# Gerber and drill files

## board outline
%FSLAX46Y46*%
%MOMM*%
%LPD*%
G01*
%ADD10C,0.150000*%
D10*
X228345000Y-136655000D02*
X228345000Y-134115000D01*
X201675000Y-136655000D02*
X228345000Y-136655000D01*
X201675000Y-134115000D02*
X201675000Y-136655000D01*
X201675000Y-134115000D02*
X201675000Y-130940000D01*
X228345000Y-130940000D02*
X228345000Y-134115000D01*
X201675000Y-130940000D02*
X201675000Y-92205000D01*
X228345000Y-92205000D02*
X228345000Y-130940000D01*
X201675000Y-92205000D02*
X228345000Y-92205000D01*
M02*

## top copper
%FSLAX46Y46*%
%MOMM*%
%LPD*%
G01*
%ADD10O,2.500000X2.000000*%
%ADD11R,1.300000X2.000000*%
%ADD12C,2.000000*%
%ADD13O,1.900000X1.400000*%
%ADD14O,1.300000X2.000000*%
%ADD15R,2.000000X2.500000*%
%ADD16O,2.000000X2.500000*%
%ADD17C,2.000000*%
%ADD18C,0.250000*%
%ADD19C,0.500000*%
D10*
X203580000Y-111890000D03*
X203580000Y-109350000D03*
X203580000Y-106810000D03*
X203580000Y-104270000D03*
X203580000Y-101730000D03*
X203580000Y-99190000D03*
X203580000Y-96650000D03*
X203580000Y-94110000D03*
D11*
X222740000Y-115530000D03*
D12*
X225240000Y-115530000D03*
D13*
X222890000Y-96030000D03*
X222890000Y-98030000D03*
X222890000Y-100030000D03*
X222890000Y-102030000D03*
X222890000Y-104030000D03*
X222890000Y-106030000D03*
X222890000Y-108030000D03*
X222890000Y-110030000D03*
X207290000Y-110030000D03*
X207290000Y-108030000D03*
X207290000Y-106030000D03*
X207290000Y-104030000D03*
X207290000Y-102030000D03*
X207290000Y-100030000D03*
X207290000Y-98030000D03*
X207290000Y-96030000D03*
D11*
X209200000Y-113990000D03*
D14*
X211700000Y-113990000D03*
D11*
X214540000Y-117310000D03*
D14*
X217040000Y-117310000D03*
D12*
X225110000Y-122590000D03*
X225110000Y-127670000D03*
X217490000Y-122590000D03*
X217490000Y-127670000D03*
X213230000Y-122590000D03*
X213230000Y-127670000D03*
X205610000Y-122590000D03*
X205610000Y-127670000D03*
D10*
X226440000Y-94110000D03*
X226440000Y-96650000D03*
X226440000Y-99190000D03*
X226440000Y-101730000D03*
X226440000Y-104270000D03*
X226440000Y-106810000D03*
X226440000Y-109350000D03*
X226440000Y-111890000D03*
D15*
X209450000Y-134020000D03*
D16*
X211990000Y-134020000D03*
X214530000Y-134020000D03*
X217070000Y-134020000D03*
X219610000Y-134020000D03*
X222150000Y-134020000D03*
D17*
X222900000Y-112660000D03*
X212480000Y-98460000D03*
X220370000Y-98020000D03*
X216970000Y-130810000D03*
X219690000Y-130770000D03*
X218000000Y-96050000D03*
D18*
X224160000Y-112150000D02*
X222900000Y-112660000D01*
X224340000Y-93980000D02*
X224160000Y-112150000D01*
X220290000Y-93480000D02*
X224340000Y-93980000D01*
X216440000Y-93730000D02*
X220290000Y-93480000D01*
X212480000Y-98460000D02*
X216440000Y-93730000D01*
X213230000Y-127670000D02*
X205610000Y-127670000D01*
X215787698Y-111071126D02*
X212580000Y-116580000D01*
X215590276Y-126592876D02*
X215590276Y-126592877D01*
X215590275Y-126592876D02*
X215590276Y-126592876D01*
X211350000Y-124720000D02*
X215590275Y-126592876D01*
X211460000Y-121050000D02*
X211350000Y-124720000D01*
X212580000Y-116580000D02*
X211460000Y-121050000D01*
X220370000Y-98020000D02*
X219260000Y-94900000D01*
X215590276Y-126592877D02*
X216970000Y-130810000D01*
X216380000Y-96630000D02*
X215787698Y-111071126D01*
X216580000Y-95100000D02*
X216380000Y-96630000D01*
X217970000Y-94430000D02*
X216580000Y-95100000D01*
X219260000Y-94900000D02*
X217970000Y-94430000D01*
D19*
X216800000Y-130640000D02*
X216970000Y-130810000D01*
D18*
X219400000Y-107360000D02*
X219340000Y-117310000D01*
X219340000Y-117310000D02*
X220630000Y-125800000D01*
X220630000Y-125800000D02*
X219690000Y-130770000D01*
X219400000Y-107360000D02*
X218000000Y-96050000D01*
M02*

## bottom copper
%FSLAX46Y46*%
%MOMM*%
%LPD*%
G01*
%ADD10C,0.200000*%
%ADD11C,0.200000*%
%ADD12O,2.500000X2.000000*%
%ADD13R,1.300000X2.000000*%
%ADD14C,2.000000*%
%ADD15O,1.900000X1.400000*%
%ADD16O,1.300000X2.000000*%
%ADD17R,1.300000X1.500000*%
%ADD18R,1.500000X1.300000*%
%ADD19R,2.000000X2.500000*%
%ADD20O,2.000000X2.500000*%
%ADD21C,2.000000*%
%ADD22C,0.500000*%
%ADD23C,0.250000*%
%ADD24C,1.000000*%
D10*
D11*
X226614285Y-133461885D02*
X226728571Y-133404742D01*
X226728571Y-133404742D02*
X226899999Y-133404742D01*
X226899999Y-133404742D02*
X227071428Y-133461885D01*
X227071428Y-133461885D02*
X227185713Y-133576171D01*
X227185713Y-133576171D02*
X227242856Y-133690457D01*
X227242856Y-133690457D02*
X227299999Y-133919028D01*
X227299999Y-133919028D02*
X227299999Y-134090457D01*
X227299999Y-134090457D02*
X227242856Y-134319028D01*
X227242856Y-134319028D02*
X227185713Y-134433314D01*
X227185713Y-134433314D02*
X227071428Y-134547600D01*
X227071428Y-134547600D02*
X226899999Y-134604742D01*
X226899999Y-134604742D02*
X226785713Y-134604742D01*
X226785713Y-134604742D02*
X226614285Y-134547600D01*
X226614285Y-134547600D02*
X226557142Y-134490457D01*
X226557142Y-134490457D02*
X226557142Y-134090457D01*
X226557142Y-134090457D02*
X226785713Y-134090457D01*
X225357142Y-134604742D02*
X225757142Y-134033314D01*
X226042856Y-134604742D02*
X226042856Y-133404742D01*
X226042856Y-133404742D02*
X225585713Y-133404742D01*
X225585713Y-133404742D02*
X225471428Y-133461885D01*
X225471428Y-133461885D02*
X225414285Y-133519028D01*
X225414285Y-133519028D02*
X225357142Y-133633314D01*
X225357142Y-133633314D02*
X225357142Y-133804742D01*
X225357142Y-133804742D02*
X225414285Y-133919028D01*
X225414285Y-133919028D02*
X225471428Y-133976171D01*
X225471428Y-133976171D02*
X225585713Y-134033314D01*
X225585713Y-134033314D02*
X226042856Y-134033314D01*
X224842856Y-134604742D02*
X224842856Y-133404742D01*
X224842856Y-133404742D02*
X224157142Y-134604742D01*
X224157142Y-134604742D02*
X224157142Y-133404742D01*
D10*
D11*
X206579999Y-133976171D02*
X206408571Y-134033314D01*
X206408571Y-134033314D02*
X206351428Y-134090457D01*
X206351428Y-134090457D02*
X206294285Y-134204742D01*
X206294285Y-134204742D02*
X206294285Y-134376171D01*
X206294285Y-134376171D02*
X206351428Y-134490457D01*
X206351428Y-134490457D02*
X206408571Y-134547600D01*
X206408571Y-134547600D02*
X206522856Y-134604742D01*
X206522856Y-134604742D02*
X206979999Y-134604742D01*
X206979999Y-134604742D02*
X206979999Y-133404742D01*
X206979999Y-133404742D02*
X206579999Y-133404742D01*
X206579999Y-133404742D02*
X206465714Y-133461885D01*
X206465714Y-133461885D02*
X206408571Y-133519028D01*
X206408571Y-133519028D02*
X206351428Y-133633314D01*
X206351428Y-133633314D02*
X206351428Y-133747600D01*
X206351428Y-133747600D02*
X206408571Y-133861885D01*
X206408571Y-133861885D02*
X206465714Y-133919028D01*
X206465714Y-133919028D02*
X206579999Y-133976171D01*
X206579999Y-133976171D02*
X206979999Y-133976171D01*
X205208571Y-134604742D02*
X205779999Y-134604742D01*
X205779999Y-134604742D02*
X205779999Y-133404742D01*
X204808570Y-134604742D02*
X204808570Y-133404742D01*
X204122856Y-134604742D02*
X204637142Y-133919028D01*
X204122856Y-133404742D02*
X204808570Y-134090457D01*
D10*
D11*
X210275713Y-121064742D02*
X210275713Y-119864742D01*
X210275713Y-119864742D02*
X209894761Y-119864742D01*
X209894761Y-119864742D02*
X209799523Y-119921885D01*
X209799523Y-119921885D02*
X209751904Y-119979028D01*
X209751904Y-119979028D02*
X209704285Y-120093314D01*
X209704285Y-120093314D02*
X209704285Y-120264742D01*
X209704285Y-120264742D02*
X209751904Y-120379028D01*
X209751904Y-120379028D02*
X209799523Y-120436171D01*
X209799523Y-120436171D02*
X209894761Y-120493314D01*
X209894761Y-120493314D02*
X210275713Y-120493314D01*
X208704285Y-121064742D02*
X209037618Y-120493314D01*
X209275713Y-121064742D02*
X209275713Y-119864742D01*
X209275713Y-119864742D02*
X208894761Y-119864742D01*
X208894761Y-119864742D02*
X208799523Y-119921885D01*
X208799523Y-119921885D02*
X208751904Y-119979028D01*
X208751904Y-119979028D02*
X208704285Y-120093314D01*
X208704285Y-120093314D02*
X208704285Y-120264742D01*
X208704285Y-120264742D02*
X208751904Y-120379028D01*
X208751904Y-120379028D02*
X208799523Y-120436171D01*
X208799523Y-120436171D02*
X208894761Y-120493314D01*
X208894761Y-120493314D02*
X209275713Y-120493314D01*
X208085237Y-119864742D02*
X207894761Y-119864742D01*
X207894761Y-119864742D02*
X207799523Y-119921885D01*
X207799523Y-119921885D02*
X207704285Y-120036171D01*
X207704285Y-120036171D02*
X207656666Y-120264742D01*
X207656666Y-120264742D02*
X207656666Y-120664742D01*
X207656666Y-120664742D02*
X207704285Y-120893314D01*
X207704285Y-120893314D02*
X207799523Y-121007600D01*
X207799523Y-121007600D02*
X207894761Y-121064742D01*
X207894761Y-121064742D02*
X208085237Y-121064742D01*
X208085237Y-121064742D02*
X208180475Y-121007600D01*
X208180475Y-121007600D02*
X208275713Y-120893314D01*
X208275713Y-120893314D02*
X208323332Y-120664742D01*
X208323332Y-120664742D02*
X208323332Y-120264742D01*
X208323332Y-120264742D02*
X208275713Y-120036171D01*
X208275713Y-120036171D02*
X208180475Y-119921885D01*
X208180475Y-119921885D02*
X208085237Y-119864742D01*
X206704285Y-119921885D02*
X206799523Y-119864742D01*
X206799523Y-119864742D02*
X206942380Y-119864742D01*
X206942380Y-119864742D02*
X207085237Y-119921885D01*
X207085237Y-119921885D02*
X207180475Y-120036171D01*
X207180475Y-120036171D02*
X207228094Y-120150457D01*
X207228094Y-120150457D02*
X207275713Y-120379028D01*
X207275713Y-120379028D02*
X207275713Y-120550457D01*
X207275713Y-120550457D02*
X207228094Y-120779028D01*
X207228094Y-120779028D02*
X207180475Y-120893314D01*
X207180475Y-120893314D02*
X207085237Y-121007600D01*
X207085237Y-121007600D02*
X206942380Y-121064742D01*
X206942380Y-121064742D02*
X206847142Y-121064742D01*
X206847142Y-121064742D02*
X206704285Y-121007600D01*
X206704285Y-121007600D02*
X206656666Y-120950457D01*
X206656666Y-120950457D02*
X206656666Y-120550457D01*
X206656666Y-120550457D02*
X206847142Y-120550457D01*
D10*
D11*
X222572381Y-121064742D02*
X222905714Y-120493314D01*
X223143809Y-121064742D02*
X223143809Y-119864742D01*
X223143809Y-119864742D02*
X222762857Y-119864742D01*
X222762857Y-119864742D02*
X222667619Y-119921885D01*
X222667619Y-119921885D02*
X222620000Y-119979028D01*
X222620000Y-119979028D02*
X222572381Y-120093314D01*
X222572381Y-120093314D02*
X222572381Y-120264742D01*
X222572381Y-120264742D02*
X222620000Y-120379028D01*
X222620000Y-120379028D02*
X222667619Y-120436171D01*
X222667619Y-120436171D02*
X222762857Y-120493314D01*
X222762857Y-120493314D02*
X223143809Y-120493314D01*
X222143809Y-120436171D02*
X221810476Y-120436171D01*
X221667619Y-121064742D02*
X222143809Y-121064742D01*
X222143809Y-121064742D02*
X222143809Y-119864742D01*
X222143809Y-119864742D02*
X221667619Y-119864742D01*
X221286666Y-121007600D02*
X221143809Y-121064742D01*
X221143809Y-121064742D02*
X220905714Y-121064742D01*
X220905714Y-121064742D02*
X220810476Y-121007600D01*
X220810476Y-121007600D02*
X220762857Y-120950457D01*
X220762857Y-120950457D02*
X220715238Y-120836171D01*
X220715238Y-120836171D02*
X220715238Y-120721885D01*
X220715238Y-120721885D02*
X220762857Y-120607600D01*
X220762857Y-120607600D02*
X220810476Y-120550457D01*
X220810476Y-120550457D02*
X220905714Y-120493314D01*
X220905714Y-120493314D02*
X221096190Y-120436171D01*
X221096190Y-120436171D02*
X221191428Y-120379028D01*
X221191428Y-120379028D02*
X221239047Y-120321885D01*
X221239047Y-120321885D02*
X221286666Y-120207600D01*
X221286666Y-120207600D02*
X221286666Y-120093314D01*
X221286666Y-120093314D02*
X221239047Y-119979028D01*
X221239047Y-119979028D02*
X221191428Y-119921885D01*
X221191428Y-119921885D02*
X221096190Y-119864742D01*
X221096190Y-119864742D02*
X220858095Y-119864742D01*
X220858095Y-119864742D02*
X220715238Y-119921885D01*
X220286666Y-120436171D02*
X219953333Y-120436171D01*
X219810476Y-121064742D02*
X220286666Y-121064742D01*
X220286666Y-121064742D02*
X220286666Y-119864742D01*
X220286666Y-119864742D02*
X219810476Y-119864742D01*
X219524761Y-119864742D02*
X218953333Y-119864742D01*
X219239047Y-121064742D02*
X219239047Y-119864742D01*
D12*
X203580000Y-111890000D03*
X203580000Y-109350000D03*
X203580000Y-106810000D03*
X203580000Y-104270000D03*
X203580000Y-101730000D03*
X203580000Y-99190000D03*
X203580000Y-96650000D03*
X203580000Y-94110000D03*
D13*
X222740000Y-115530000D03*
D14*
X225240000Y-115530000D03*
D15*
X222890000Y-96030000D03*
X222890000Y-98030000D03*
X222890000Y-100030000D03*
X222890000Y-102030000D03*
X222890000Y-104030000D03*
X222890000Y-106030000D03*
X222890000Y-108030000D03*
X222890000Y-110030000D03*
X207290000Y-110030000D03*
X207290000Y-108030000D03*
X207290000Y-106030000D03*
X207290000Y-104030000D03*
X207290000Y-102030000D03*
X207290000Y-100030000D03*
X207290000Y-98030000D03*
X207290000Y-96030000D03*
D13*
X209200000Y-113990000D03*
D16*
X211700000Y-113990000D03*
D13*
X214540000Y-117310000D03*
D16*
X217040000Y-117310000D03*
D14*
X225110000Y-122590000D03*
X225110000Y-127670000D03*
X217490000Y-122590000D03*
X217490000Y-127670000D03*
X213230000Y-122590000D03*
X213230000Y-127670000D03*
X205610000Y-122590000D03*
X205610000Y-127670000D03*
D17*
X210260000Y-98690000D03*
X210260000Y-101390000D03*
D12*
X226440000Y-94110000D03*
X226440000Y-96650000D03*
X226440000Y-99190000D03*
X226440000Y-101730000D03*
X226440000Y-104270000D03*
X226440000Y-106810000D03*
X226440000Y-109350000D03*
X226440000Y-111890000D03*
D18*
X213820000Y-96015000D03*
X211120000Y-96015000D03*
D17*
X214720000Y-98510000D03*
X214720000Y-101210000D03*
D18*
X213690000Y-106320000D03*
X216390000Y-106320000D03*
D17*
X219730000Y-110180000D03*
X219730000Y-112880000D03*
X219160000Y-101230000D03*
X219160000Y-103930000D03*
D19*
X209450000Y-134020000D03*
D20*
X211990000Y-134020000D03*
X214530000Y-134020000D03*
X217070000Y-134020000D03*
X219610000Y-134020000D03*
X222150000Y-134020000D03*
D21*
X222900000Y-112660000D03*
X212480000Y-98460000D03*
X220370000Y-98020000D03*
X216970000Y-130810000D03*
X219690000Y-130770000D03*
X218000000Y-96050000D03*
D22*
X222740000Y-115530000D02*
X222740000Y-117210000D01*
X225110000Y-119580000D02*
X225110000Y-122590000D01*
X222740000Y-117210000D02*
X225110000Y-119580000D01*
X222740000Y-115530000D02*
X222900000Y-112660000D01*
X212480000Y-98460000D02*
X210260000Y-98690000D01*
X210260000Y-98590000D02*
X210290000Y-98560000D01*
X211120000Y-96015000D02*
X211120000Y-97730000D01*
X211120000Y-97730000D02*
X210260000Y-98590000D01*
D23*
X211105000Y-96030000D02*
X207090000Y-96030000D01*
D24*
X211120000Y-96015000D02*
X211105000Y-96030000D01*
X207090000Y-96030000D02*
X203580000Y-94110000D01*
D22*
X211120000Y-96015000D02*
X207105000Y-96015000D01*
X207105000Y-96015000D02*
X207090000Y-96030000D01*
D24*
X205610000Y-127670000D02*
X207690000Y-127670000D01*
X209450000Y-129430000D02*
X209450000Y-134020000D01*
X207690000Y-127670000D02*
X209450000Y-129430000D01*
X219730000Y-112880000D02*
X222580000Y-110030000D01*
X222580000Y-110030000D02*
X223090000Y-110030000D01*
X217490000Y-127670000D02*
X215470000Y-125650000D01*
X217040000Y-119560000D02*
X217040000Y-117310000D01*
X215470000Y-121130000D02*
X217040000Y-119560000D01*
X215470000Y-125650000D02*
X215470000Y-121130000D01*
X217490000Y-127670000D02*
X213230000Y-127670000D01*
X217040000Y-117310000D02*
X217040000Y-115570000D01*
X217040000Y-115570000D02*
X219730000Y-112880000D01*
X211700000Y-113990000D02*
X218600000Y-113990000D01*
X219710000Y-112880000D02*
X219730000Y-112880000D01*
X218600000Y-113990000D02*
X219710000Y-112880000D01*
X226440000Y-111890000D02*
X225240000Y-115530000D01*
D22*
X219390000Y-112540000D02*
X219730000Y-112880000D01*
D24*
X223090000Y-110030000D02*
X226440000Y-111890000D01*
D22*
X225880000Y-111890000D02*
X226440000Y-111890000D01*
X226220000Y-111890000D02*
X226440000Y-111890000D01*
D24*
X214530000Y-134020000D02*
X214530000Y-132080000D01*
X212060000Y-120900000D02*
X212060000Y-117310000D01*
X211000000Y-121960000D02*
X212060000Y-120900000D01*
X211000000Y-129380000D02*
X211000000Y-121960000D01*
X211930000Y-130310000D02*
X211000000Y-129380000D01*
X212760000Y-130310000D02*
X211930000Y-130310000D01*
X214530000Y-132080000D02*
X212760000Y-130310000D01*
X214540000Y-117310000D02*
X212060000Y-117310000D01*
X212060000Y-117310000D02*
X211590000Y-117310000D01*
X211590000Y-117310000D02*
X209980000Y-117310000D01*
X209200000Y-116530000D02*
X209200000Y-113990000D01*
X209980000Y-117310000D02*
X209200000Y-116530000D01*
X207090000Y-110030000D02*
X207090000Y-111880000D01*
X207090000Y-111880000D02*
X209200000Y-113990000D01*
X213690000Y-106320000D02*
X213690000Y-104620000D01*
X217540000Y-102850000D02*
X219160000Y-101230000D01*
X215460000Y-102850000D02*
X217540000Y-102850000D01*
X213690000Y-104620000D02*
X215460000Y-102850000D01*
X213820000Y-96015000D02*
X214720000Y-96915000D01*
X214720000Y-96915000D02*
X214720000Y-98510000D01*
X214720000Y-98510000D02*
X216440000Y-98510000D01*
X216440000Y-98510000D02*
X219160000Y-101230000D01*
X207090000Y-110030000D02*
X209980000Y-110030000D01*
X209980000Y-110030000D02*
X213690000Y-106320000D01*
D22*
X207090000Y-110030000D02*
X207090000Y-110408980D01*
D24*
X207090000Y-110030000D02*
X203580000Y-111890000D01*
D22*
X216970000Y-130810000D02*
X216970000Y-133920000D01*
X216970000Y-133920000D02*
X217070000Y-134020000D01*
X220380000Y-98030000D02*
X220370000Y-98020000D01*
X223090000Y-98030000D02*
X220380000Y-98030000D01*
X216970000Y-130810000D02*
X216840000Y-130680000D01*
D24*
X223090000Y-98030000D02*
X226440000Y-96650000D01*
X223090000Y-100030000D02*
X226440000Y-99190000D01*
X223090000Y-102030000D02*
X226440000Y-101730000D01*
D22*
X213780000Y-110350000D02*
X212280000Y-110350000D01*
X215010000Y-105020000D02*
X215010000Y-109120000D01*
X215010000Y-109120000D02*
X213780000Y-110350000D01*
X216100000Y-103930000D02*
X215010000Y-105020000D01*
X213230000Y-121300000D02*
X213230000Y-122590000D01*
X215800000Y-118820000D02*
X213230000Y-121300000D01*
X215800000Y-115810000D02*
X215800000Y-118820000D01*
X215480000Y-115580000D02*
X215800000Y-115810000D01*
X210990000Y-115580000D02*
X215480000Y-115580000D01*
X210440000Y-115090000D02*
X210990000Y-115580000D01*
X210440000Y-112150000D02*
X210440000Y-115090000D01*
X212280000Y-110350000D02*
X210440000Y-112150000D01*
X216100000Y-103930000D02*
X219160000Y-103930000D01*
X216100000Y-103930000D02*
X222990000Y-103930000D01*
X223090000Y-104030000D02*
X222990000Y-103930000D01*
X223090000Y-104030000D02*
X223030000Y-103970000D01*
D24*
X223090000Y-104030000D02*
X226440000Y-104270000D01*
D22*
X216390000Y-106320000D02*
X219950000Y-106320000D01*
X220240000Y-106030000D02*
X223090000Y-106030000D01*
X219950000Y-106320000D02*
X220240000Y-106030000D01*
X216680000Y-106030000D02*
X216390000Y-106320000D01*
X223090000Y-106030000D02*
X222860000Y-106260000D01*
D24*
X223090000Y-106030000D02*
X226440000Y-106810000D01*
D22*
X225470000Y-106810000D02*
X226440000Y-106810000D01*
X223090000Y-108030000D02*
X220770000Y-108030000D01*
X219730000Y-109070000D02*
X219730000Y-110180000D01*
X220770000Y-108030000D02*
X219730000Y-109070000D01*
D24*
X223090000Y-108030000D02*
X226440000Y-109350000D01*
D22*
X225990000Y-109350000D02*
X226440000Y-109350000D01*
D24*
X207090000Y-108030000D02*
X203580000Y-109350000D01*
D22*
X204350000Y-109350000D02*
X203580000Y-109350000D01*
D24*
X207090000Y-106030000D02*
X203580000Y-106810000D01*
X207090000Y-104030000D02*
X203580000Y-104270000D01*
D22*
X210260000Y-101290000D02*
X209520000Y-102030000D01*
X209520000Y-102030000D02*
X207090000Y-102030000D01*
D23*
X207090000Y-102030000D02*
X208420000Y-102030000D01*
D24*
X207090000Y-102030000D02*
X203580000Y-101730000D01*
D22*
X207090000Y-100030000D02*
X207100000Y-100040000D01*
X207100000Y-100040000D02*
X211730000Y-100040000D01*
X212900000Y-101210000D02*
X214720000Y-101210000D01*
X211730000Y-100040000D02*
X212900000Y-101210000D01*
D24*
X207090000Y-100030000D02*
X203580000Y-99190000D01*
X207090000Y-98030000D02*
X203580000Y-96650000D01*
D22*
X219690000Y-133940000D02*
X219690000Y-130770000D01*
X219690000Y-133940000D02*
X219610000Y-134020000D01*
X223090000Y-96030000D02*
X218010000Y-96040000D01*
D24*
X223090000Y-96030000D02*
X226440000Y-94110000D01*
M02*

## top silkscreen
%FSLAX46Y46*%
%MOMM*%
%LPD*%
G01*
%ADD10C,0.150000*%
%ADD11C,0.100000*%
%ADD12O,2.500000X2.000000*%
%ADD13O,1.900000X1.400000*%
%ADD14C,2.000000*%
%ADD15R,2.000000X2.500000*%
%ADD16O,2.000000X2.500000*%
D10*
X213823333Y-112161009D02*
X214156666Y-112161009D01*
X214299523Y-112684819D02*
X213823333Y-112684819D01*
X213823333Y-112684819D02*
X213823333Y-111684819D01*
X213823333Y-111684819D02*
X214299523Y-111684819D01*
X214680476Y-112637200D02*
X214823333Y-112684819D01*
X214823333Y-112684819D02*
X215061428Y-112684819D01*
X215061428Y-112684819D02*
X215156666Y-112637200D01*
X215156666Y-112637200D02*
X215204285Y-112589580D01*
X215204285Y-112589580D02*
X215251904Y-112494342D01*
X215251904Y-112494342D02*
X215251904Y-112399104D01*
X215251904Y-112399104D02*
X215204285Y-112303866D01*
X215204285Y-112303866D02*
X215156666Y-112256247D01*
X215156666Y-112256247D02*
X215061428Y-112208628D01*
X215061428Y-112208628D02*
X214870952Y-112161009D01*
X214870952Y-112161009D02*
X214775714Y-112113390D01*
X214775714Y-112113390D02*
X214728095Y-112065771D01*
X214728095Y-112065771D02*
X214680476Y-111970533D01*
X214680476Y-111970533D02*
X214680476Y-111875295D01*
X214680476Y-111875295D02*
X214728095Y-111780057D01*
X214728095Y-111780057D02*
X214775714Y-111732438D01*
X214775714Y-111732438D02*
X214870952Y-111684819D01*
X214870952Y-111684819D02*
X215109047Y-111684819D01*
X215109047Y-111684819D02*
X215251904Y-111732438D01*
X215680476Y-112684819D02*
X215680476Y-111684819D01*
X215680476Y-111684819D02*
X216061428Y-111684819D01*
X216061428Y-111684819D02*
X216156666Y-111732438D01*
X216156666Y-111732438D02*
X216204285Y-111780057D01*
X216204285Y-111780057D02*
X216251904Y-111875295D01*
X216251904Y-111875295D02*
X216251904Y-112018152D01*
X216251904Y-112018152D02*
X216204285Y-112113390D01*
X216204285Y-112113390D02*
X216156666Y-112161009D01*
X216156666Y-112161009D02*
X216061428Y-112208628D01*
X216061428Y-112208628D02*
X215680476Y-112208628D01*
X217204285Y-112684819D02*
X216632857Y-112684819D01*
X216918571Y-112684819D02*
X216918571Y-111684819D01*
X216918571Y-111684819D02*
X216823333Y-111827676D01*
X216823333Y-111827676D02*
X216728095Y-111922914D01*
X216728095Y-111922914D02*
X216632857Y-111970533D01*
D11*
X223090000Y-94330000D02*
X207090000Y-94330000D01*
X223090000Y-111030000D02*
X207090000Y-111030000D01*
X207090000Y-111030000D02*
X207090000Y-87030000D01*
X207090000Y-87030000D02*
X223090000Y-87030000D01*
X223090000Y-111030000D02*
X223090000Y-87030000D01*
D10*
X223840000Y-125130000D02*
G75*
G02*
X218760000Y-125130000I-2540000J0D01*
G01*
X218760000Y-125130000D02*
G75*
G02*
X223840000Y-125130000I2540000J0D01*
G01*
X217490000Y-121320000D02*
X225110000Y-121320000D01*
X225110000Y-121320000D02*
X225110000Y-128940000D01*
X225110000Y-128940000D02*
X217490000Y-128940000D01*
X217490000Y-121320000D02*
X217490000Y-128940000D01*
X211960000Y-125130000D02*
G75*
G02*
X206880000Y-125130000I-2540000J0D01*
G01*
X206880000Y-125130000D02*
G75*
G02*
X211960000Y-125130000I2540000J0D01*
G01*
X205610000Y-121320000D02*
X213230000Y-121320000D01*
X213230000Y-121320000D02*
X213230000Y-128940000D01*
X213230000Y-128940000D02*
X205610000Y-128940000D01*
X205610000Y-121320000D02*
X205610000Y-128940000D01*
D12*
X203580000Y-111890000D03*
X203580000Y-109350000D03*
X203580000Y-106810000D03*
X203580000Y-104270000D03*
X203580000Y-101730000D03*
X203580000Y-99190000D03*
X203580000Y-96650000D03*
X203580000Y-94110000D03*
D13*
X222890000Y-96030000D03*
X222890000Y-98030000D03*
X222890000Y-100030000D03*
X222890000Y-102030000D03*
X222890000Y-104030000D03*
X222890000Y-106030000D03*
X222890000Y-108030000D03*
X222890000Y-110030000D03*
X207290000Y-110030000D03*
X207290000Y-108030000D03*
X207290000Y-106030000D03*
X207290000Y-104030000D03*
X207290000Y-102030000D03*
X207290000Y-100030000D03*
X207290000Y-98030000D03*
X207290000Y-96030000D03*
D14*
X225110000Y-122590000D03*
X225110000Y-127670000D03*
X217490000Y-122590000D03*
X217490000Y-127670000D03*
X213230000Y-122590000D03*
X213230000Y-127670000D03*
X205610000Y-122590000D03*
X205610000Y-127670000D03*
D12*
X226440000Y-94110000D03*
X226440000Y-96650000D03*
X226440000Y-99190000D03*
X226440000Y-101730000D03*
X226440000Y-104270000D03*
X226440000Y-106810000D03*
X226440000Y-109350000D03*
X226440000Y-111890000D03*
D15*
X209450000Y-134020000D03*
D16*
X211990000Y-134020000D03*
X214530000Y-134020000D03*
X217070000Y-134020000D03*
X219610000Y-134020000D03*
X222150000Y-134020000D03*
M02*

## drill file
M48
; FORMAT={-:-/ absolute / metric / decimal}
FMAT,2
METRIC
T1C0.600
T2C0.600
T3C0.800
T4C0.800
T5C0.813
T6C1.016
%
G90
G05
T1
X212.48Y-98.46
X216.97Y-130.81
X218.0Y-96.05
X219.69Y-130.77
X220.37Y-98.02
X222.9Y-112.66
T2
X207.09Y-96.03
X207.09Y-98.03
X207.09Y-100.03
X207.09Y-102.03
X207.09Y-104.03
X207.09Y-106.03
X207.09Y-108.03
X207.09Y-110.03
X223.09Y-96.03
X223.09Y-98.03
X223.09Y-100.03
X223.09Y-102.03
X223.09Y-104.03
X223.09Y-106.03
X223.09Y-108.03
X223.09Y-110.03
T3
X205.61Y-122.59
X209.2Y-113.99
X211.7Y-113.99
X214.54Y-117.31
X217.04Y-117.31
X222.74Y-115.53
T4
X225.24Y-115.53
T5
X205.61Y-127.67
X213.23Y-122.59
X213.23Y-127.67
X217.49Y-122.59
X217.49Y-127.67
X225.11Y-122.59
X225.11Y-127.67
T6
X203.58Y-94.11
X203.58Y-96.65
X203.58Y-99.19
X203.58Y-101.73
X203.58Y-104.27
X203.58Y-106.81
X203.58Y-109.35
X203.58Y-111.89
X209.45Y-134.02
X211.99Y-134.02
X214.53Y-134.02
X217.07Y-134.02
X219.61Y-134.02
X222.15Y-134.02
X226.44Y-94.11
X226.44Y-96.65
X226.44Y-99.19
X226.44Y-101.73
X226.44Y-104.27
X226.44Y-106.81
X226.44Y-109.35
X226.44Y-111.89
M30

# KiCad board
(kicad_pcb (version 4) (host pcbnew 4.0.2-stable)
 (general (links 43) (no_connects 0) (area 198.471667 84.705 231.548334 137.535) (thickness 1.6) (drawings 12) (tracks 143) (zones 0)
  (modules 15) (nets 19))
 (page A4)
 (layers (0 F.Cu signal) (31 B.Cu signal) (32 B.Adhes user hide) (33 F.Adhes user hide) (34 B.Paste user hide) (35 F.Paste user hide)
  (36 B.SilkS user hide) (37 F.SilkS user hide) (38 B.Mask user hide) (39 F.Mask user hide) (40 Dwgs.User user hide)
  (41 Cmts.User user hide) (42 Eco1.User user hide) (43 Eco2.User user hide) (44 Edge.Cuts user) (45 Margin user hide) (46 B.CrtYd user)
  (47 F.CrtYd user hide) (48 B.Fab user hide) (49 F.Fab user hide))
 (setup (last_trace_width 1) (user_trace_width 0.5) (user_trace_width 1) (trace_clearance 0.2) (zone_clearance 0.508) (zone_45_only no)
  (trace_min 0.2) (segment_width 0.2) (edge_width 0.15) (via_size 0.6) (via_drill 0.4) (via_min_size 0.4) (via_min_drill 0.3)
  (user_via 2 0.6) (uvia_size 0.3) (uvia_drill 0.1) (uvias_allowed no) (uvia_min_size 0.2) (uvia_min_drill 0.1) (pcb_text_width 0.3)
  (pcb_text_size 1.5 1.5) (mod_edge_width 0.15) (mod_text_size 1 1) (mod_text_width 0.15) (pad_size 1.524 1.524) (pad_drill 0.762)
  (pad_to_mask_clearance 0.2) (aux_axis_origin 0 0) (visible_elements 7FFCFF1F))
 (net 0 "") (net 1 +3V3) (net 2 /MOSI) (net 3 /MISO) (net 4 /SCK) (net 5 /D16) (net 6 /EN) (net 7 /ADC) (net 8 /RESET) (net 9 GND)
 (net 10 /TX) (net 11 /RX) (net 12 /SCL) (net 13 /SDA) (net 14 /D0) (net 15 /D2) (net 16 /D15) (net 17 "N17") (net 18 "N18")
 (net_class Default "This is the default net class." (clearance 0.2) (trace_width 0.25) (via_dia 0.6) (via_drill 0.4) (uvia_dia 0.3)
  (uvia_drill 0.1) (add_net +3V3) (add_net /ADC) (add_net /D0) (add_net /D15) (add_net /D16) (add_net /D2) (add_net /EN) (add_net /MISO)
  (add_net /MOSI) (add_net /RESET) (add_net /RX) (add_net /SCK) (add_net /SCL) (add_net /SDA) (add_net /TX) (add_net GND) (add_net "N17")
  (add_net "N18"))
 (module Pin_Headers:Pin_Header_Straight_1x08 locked (layer F.Cu) (at 203.58 111.89 180)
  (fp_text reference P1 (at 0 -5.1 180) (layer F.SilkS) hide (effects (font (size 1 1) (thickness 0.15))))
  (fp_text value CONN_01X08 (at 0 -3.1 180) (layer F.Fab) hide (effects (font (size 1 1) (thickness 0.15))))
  (pad 1 thru_hole oval (at 0 0 180) (size 2.5 2) (drill 1.016) (layers *.Cu *.Mask F.SilkS) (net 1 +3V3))
  (pad 2 thru_hole oval (at 0 2.54 180) (size 2.5 2) (drill 1.016) (layers *.Cu *.Mask F.SilkS) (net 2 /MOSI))
  (pad 3 thru_hole oval (at 0 5.08 180) (size 2.5 2) (drill 1.016) (layers *.Cu *.Mask F.SilkS) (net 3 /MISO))
  (pad 4 thru_hole oval (at 0 7.62 180) (size 2.5 2) (drill 1.016) (layers *.Cu *.Mask F.SilkS) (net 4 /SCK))
  (pad 5 thru_hole oval (at 0 10.16 180) (size 2.5 2) (drill 1.016) (layers *.Cu *.Mask F.SilkS) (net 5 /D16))
  (pad 6 thru_hole oval (at 0 12.7 180) (size 2.5 2) (drill 1.016) (layers *.Cu *.Mask F.SilkS) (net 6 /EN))
  (pad 7 thru_hole oval (at 0 15.24 180) (size 2.5 2) (drill 1.016) (layers *.Cu *.Mask F.SilkS) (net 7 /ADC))
  (pad 8 thru_hole oval (at 0 17.78 180) (size 2.5 2) (drill 1.016) (layers *.Cu *.Mask F.SilkS) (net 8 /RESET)))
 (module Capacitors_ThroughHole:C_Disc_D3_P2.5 (layer B.Cu) (at 222.74 115.53)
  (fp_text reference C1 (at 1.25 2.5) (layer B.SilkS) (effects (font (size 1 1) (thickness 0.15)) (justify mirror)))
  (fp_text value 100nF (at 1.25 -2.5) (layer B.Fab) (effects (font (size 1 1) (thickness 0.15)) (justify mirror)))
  (pad 1 thru_hole rect (at 0 0) (size 1.3 2) (drill 0.8) (layers *.Cu *.Mask B.SilkS) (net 8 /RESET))
  (pad 2 thru_hole circle (at 2.5 0) (size 2 2) (drill 0.8001) (layers *.Cu *.Mask B.SilkS) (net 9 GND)))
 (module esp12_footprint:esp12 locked (layer F.Cu) (at 207.09 92.03)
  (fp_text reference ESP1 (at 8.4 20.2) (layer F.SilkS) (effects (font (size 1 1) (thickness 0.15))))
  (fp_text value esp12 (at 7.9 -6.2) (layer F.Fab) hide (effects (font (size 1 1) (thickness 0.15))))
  (fp_line (start 16 2.3) (end 0 2.3) (layer F.SilkS) (width 0.1))
  (fp_line (start 16 19) (end 0 19) (layer F.SilkS) (width 0.1))
  (fp_line (start 0 19) (end 0 -5) (layer F.SilkS) (width 0.1))
  (fp_line (start 0 -5) (end 16 -5) (layer F.SilkS) (width 0.1))
  (fp_line (start 16 19) (end 16 -5) (layer F.SilkS) (width 0.1))
  (pad 16 thru_hole oval (at 16 4 180) (size 1.9 1.4) (drill 0.6 (offset 0.2 0)) (layers *.Cu *.Mask F.SilkS) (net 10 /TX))
  (pad 15 thru_hole oval (at 16 6 180) (size 1.9 1.4) (drill 0.6 (offset 0.2 0)) (layers *.Cu *.Mask F.SilkS) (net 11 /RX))
  (pad 14 thru_hole oval (at 16 8 180) (size 1.9 1.4) (drill 0.6 (offset 0.2 0)) (layers *.Cu *.Mask F.SilkS) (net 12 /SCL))
  (pad 13 thru_hole oval (at 16 10 180) (size 1.9 1.4) (drill 0.6 (offset 0.2 0)) (layers *.Cu *.Mask F.SilkS) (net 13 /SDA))
  (pad 12 thru_hole oval (at 16 12 180) (size 1.9 1.4) (drill 0.6 (offset 0.2 0)) (layers *.Cu *.Mask F.SilkS) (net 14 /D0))
  (pad 11 thru_hole oval (at 16 14 180) (size 1.9 1.4) (drill 0.6 (offset 0.2 0)) (layers *.Cu *.Mask F.SilkS) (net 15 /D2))
  (pad 10 thru_hole oval (at 16 16 180) (size 1.9 1.4) (drill 0.6 (offset 0.2 0)) (layers *.Cu *.Mask F.SilkS) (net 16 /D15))
  (pad 9 thru_hole oval (at 16 18 180) (size 1.9 1.4) (drill 0.6 (offset 0.2 0)) (layers *.Cu *.Mask F.SilkS) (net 9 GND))
  (pad 8 thru_hole oval (at 0 18) (size 1.9 1.4) (drill 0.6 (offset 0.2 0)) (layers *.Cu *.Mask F.SilkS) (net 1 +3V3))
  (pad 7 thru_hole oval (at 0 16) (size 1.9 1.4) (drill 0.6 (offset 0.2 0)) (layers *.Cu *.Mask F.SilkS) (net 2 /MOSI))
  (pad 6 thru_hole oval (at 0 14) (size 1.9 1.4) (drill 0.6 (offset 0.2 0)) (layers *.Cu *.Mask F.SilkS) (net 3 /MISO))
  (pad 5 thru_hole oval (at 0 12) (size 1.9 1.4) (drill 0.6 (offset 0.2 0)) (layers *.Cu *.Mask F.SilkS) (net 4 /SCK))
  (pad 4 thru_hole oval (at 0 10) (size 1.9 1.4) (drill 0.6 (offset 0.2 0)) (layers *.Cu *.Mask F.SilkS) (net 5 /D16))
  (pad 3 thru_hole oval (at 0 8) (size 1.9 1.4) (drill 0.6 (offset 0.2 0)) (layers *.Cu *.Mask F.SilkS) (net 6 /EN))
  (pad 2 thru_hole oval (at 0 6) (size 1.9 1.4) (drill 0.6 (offset 0.2 0)) (layers *.Cu *.Mask F.SilkS) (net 7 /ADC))
  (pad 1 thru_hole oval (at 0 4) (size 1.9 1.4) (drill 0.6 (offset 0.2 0)) (layers *.Cu *.Mask F.SilkS) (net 8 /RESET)))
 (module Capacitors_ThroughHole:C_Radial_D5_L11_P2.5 (layer B.Cu) (at 209.2 113.99)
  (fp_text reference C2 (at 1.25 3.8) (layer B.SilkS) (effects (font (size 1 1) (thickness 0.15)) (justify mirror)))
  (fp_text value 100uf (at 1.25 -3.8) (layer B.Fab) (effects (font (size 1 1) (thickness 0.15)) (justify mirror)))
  (pad 1 thru_hole rect (at 0 0) (size 1.3 2) (drill 0.8) (layers *.Cu *.Mask B.SilkS) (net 1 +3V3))
  (pad 2 thru_hole oval (at 2.5 0) (size 1.3 2) (drill 0.8) (layers *.Cu *.Mask B.SilkS) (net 9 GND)))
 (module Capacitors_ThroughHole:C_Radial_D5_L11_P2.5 (layer B.Cu) (at 214.54 117.31)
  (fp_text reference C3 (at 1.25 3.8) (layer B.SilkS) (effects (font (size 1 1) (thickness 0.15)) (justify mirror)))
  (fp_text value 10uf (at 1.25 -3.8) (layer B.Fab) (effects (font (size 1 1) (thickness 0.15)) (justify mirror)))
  (pad 1 thru_hole rect (at 0 0) (size 1.3 2) (drill 0.8) (layers *.Cu *.Mask B.SilkS) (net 1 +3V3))
  (pad 2 thru_hole oval (at 2.5 0) (size 1.3 2) (drill 0.8) (layers *.Cu *.Mask B.SilkS) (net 9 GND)))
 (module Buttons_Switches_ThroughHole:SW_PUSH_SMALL (layer F.Cu) (at 221.3 125.13)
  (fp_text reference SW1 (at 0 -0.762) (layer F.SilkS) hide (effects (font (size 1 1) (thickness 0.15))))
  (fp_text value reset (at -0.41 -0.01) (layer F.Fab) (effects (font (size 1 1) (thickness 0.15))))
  (fp_circle (center 0 0) (end 0 -2.54) (layer F.SilkS) (width 0.15))
  (fp_line (start -3.81 -3.81) (end 3.81 -3.81) (layer F.SilkS) (width 0.15))
  (fp_line (start 3.81 -3.81) (end 3.81 3.81) (layer F.SilkS) (width 0.15))
  (fp_line (start 3.81 3.81) (end -3.81 3.81) (layer F.SilkS) (width 0.15))
  (fp_line (start -3.81 -3.81) (end -3.81 3.81) (layer F.SilkS) (width 0.15))
  (pad 1 thru_hole circle (at 3.81 -2.54) (size 2 2) (drill 0.8128) (layers *.Cu *.Mask F.SilkS) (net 8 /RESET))
  (pad X thru_hole circle (at 3.81 2.54) (size 2 2) (drill 0.8128) (layers *.Cu *.Mask F.SilkS))
  (pad X thru_hole circle (at -3.81 -2.54) (size 2 2) (drill 0.8128) (layers *.Cu *.Mask F.SilkS))
  (pad 2 thru_hole circle (at -3.81 2.54) (size 2 2) (drill 0.8128) (layers *.Cu *.Mask F.SilkS) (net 9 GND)))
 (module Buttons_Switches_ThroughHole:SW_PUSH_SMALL (layer F.Cu) (at 209.42 125.13)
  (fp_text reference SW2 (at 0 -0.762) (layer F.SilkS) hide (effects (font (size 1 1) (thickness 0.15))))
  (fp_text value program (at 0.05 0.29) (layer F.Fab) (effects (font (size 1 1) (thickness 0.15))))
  (fp_circle (center 0 0) (end 0 -2.54) (layer F.SilkS) (width 0.15))
  (fp_line (start -3.81 -3.81) (end 3.81 -3.81) (layer F.SilkS) (width 0.15))
  (fp_line (start 3.81 -3.81) (end 3.81 3.81) (layer F.SilkS) (width 0.15))
  (fp_line (start 3.81 3.81) (end -3.81 3.81) (layer F.SilkS) (width 0.15))
  (fp_line (start -3.81 -3.81) (end -3.81 3.81) (layer F.SilkS) (width 0.15))
  (pad 1 thru_hole circle (at 3.81 -2.54) (size 2 2) (drill 0.8128) (layers *.Cu *.Mask F.SilkS) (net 14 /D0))
  (pad 2 thru_hole circle (at 3.81 2.54) (size 2 2) (drill 0.8128) (layers *.Cu *.Mask F.SilkS) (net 9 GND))
  (pad X thru_hole circle (at -3.81 -2.54) (size 2 2) (drill 0.8) (layers *.Cu *.Mask F.SilkS))
  (pad 2 thru_hole circle (at -3.81 2.54) (size 2 2) (drill 0.8128) (layers *.Cu *.Mask F.SilkS) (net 9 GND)))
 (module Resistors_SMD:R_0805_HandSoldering (layer B.Cu) (at 210.26 100.04 270)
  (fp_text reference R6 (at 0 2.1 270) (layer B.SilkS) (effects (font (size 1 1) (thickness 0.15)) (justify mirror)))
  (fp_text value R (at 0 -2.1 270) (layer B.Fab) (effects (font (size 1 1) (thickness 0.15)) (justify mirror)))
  (pad 1 smd rect (at -1.35 0 270) (size 1.5 1.3) (layers B.Cu B.Paste B.Mask) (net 8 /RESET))
  (pad 2 smd rect (at 1.35 0 270) (size 1.5 1.3) (layers B.Cu B.Paste B.Mask) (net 5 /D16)))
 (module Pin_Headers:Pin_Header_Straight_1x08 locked (layer F.Cu) (at 226.44 94.11)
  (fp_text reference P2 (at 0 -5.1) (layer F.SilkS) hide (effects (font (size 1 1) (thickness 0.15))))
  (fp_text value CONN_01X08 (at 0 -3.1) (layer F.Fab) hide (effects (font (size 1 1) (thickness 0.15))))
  (pad 1 thru_hole oval (at 0 0) (size 2.5 2) (drill 1.016) (layers *.Cu *.Mask F.SilkS) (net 10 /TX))
  (pad 2 thru_hole oval (at 0 2.54) (size 2.5 2) (drill 1.016) (layers *.Cu *.Mask F.SilkS) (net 11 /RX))
  (pad 3 thru_hole oval (at 0 5.08) (size 2.5 2) (drill 1.016) (layers *.Cu *.Mask F.SilkS) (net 12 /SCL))
  (pad 4 thru_hole oval (at 0 7.62) (size 2.5 2) (drill 1.016) (layers *.Cu *.Mask F.SilkS) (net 13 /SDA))
  (pad 5 thru_hole oval (at 0 10.16) (size 2.5 2) (drill 1.016) (layers *.Cu *.Mask F.SilkS) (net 14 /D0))
  (pad 6 thru_hole oval (at 0 12.7) (size 2.5 2) (drill 1.016) (layers *.Cu *.Mask F.SilkS) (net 15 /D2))
  (pad 7 thru_hole oval (at 0 15.24) (size 2.5 2) (drill 1.016) (layers *.Cu *.Mask F.SilkS) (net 16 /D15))
  (pad 8 thru_hole oval (at 0 17.78) (size 2.5 2) (drill 1.016) (layers *.Cu *.Mask F.SilkS) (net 9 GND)))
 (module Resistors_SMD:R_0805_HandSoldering (layer B.Cu) (at 212.47 96.015 180)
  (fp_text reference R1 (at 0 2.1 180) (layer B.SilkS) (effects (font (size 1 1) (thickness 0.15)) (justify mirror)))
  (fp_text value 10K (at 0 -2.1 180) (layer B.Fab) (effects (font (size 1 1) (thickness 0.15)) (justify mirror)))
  (pad 1 smd rect (at -1.35 0 180) (size 1.5 1.3) (layers B.Cu B.Paste B.Mask) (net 1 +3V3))
  (pad 2 smd rect (at 1.35 0 180) (size 1.5 1.3) (layers B.Cu B.Paste B.Mask) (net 8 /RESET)))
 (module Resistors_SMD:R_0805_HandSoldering (layer B.Cu) (at 214.72 99.86 270)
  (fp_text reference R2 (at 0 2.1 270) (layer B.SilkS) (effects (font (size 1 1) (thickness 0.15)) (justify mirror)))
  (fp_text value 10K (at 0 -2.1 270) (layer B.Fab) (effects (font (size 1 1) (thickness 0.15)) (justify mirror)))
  (pad 1 smd rect (at -1.35 0 270) (size 1.5 1.3) (layers B.Cu B.Paste B.Mask) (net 1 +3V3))
  (pad 2 smd rect (at 1.35 0 270) (size 1.5 1.3) (layers B.Cu B.Paste B.Mask) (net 6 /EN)))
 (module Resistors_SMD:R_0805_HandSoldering (layer B.Cu) (at 215.04 106.32)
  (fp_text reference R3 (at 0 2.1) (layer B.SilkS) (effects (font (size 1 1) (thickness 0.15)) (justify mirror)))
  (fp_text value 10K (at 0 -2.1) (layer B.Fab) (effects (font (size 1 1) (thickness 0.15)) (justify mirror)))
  (pad 1 smd rect (at -1.35 0) (size 1.5 1.3) (layers B.Cu B.Paste B.Mask) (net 1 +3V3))
  (pad 2 smd rect (at 1.35 0) (size 1.5 1.3) (layers B.Cu B.Paste B.Mask) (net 15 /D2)))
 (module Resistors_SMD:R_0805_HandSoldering (layer B.Cu) (at 219.73 111.53 270)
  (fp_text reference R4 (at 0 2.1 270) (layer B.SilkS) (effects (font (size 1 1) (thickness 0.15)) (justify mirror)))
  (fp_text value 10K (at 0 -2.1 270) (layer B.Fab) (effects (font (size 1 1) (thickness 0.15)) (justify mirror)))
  (pad 1 smd rect (at -1.35 0 270) (size 1.5 1.3) (layers B.Cu B.Paste B.Mask) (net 16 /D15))
  (pad 2 smd rect (at 1.35 0 270) (size 1.5 1.3) (layers B.Cu B.Paste B.Mask) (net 9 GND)))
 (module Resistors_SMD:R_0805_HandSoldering (layer B.Cu) (at 219.16 102.58 270)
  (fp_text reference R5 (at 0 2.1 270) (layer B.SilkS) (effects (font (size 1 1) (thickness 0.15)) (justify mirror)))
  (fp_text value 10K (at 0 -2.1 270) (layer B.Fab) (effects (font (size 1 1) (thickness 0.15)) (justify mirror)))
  (pad 1 smd rect (at -1.35 0 270) (size 1.5 1.3) (layers B.Cu B.Paste B.Mask) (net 1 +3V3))
  (pad 2 smd rect (at 1.35 0 270) (size 1.5 1.3) (layers B.Cu B.Paste B.Mask) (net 14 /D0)))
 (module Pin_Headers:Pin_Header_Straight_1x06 (layer F.Cu) (at 209.45 134.02 90)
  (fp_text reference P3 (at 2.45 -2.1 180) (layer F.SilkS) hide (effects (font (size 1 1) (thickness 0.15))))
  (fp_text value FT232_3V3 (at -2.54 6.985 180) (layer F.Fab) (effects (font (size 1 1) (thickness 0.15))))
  (pad 1 thru_hole rect (at 0 0 90) (size 2.5 2) (drill 1.016) (layers *.Cu *.Mask F.SilkS) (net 9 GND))
  (pad 2 thru_hole oval (at 0 2.54 90) (size 2.5 2) (drill 1.016) (layers *.Cu *.Mask F.SilkS) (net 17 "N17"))
  (pad 3 thru_hole oval (at 0 5.08 90) (size 2.5 2) (drill 1.016) (layers *.Cu *.Mask F.SilkS) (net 1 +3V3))
  (pad 4 thru_hole oval (at 0 7.62 90) (size 2.5 2) (drill 1.016) (layers *.Cu *.Mask F.SilkS) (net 11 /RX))
  (pad 5 thru_hole oval (at 0 10.16 90) (size 2.5 2) (drill 1.016) (layers *.Cu *.Mask F.SilkS) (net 10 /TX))
  (pad 6 thru_hole oval (at 0 12.7 90) (size 2.5 2) (drill 1.016) (layers *.Cu *.Mask F.SilkS) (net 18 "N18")))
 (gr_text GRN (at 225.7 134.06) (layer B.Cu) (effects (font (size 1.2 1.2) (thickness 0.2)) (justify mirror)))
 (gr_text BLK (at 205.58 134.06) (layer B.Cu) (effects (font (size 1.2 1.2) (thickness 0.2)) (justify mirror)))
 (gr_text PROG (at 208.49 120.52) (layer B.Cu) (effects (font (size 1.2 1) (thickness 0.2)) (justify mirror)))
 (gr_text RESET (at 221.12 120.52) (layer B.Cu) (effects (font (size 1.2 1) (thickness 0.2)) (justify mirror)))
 (gr_line (start 228.345 136.655) (end 228.345 134.115) (angle 90) (layer Edge.Cuts) (width 0.15))
 (gr_line (start 201.675 136.655) (end 228.345 136.655) (angle 90) (layer Edge.Cuts) (width 0.15))
 (gr_line (start 201.675 134.115) (end 201.675 136.655) (angle 90) (layer Edge.Cuts) (width 0.15))
 (gr_line (start 201.675 134.115) (end 201.675 130.94) (angle 90) (layer Edge.Cuts) (width 0.15))
 (gr_line (start 228.345 130.94) (end 228.345 134.115) (angle 90) (layer Edge.Cuts) (width 0.15))
 (gr_line (start 201.675 130.94) (end 201.675 92.205) (angle 90) (layer Edge.Cuts) (width 0.15))
 (gr_line (start 228.345 92.205) (end 228.345 130.94) (angle 90) (layer Edge.Cuts) (width 0.15))
 (gr_line (start 201.675 92.205) (end 228.345 92.205) (angle 90) (layer Edge.Cuts) (width 0.15))
 (segment (start 222.74 115.53) (end 222.74 117.21) (width 0.5) (layer B.Cu) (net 8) (status 400000))
 (segment (start 225.11 119.58) (end 225.11 122.59) (width 0.5) (layer B.Cu) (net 8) (status 800000))
 (segment (start 222.74 117.21) (end 225.11 119.58) (width 0.5) (layer B.Cu) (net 8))
 (segment (start 222.74 115.53) (end 222.9 112.66) (width 0.5) (layer B.Cu) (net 8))
 (via (at 222.9 112.66) (size 2) (drill 0.6) (layers F.Cu B.Cu) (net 8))
 (segment (start 224.16 112.15) (end 222.9 112.66) (width 0.25) (layer F.Cu) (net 8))
 (segment (start 224.34 93.98) (end 224.16 112.15) (width 0.25) (layer F.Cu) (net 8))
 (segment (start 220.29 93.48) (end 224.34 93.98) (width 0.25) (layer F.Cu) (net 8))
 (segment (start 216.44 93.73) (end 220.29 93.48) (width 0.25) (layer F.Cu) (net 8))
 (segment (start 212.48 98.46) (end 216.44 93.73) (width 0.25) (layer F.Cu) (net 8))
 (via (at 212.48 98.46) (size 2) (drill 0.6) (layers F.Cu B.Cu) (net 8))
 (segment (start 212.48 98.46) (end 210.26 98.69) (width 0.5) (layer B.Cu) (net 8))
 (segment (start 210.26 98.59) (end 210.29 98.56) (width 0.5) (layer B.Cu) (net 8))
 (segment (start 211.12 96.015) (end 211.12 97.73) (width 0.5) (layer B.Cu) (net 8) (status 10))
 (segment (start 211.12 97.73) (end 210.26 98.59) (width 0.5) (layer B.Cu) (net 8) (status 20))
 (segment (start 211.105 96.03) (end 207.09 96.03) (width 0.25) (layer B.Cu) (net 8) (status 30))
 (segment (start 211.12 96.015) (end 211.105 96.03) (width 1) (layer B.Cu) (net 8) (status 30))
 (segment (start 207.09 96.03) (end 203.58 94.11) (width 1) (layer B.Cu) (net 8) (status 30))
 (segment (start 211.12 96.015) (end 207.105 96.015) (width 0.5) (layer B.Cu) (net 8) (status 30))
 (segment (start 207.105 96.015) (end 207.09 96.03) (width 0.5) (layer B.Cu) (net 8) (status 30))
 (segment (start 205.61 127.67) (end 207.69 127.67) (width 1) (layer B.Cu) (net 9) (status 400000))
 (segment (start 209.45 129.43) (end 209.45 134.02) (width 1) (layer B.Cu) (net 9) (status 800000))
 (segment (start 207.69 127.67) (end 209.45 129.43) (width 1) (layer B.Cu) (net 9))
 (segment (start 219.73 112.88) (end 222.58 110.03) (width 1) (layer B.Cu) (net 9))
 (segment (start 222.58 110.03) (end 223.09 110.03) (width 1) (layer B.Cu) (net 9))
 (segment (start 217.49 127.67) (end 215.47 125.65) (width 1) (layer B.Cu) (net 9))
 (segment (start 217.04 119.56) (end 217.04 117.31) (width 1) (layer B.Cu) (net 9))
 (segment (start 215.47 121.13) (end 217.04 119.56) (width 1) (layer B.Cu) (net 9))
 (segment (start 215.47 125.65) (end 215.47 121.13) (width 1) (layer B.Cu) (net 9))
 (segment (start 217.49 127.67) (end 213.23 127.67) (width 1) (layer B.Cu) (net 9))
 (segment (start 217.04 117.31) (end 217.04 115.57) (width 1) (layer B.Cu) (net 9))
 (segment (start 217.04 115.57) (end 219.73 112.88) (width 1) (layer B.Cu) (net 9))
 (segment (start 211.7 113.99) (end 218.6 113.99) (width 1) (layer B.Cu) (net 9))
 (segment (start 219.71 112.88) (end 219.73 112.88) (width 1) (layer B.Cu) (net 9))
 (segment (start 218.6 113.99) (end 219.71 112.88) (width 1) (layer B.Cu) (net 9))
 (segment (start 226.44 111.89) (end 225.24 115.53) (width 1) (layer B.Cu) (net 9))
 (segment (start 213.23 127.67) (end 205.61 127.67) (width 0.25) (layer F.Cu) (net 9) (status 30))
 (segment (start 219.39 112.54) (end 219.73 112.88) (width 0.5) (layer B.Cu) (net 9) (status 30))
 (segment (start 223.09 110.03) (end 226.44 111.89) (width 1) (layer B.Cu) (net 9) (status 30))
 (segment (start 225.88 111.89) (end 226.44 111.89) (width 0.5) (layer B.Cu) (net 9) (status 30))
 (segment (start 226.22 111.89) (end 226.44 111.89) (width 0.5) (layer B.Cu) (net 9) (status 30))
 (segment (start 214.53 134.02) (end 214.53 132.08) (width 1) (layer B.Cu) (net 1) (status 400000))
 (segment (start 212.06 120.9) (end 212.06 117.31) (width 1) (layer B.Cu) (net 1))
 (segment (start 211 121.96) (end 212.06 120.9) (width 1) (layer B.Cu) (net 1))
 (segment (start 211 129.38) (end 211 121.96) (width 1) (layer B.Cu) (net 1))
 (segment (start 211.93 130.31) (end 211 129.38) (width 1) (layer B.Cu) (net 1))
 (segment (start 212.76 130.31) (end 211.93 130.31) (width 1) (layer B.Cu) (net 1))
 (segment (start 214.53 132.08) (end 212.76 130.31) (width 1) (layer B.Cu) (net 1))
 (segment (start 214.54 117.31) (end 212.06 117.31) (width 1) (layer B.Cu) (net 1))
 (segment (start 212.06 117.31) (end 211.59 117.31) (width 1) (layer B.Cu) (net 1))
 (segment (start 211.59 117.31) (end 209.98 117.31) (width 1) (layer B.Cu) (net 1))
 (segment (start 209.2 116.53) (end 209.2 113.99) (width 1) (layer B.Cu) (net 1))
 (segment (start 209.98 117.31) (end 209.2 116.53) (width 1) (layer B.Cu) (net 1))
 (segment (start 207.09 110.03) (end 207.09 111.88) (width 1) (layer B.Cu) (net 1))
 (segment (start 207.09 111.88) (end 209.2 113.99) (width 1) (layer B.Cu) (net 1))
 (segment (start 213.69 106.32) (end 213.69 104.62) (width 1) (layer B.Cu) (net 1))
 (segment (start 217.54 102.85) (end 219.16 101.23) (width 1) (layer B.Cu) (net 1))
 (segment (start 215.46 102.85) (end 217.54 102.85) (width 1) (layer B.Cu) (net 1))
 (segment (start 213.69 104.62) (end 215.46 102.85) (width 1) (layer B.Cu) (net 1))
 (segment (start 213.82 96.015) (end 214.72 96.915) (width 1) (layer B.Cu) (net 1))
 (segment (start 214.72 96.915) (end 214.72 98.51) (width 1) (layer B.Cu) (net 1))
 (segment (start 214.72 98.51) (end 216.44 98.51) (width 1) (layer B.Cu) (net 1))
 (segment (start 216.44 98.51) (end 219.16 101.23) (width 1) (layer B.Cu) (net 1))
 (segment (start 207.09 110.03) (end 209.98 110.03) (width 1) (layer B.Cu) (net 1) (status 10))
 (segment (start 209.98 110.03) (end 213.69 106.32) (width 1) (layer B.Cu) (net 1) (status 20))
 (segment (start 207.09 110.03) (end 207.09 110.40898) (width 0.5) (layer B.Cu) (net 1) (status 30))
 (segment (start 207.09 110.03) (end 203.58 111.89) (width 1) (layer B.Cu) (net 1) (status 30))
 (segment (start 215.787698 111.071126) (end 212.58 116.58) (width 0.25) (layer F.Cu) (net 11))
 (segment (start 215.590276 126.592876) (end 215.590276 126.592877) (width 0.25) (layer F.Cu) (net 11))
 (segment (start 215.590275 126.592876) (end 215.590276 126.592876) (width 0.25) (layer F.Cu) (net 11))
 (segment (start 211.35 124.72) (end 215.590275 126.592876) (width 0.25) (layer F.Cu) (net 11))
 (segment (start 211.46 121.05) (end 211.35 124.72) (width 0.25) (layer F.Cu) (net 11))
 (segment (start 212.58 116.58) (end 211.46 121.05) (width 0.25) (layer F.Cu) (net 11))
 (segment (start 216.97 130.81) (end 216.97 133.92) (width 0.5) (layer B.Cu) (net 11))
 (segment (start 216.97 133.92) (end 217.07 134.02) (width 0.5) (layer B.Cu) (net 11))
 (segment (start 220.37 98.02) (end 219.26 94.9) (width 0.25) (layer F.Cu) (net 11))
 (via (at 220.37 98.02) (size 2) (drill 0.6) (layers F.Cu B.Cu) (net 11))
 (segment (start 220.38 98.03) (end 220.37 98.02) (width 0.5) (layer B.Cu) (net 11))
 (segment (start 223.09 98.03) (end 220.38 98.03) (width 0.5) (layer B.Cu) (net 11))
 (segment (start 215.590276 126.592877) (end 216.97 130.81) (width 0.25) (layer F.Cu) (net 11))
 (segment (start 216.38 96.63) (end 215.787698 111.071126) (width 0.25) (layer F.Cu) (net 11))
 (segment (start 216.58 95.1) (end 216.38 96.63) (width 0.25) (layer F.Cu) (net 11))
 (segment (start 217.97 94.43) (end 216.58 95.1) (width 0.25) (layer F.Cu) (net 11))
 (segment (start 219.26 94.9) (end 217.97 94.43) (width 0.25) (layer F.Cu) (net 11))
 (segment (start 216.97 130.81) (end 216.84 130.68) (width 0.5) (layer B.Cu) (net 11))
 (segment (start 216.8 130.64) (end 216.97 130.81) (width 0.5) (layer F.Cu) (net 11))
 (via (at 216.97 130.81) (size 2) (drill 0.6) (layers F.Cu B.Cu) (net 11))
 (segment (start 223.09 98.03) (end 226.44 96.65) (width 1) (layer B.Cu) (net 11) (status 30))
 (segment (start 223.09 100.03) (end 226.44 99.19) (width 1) (layer B.Cu) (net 12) (status 30))
 (segment (start 223.09 102.03) (end 226.44 101.73) (width 1) (layer B.Cu) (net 13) (status 30))
 (segment (start 213.78 110.35) (end 212.28 110.35) (width 0.5) (layer B.Cu) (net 14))
 (segment (start 215.01 105.02) (end 215.01 109.12) (width 0.5) (layer B.Cu) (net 14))
 (segment (start 215.01 109.12) (end 213.78 110.35) (width 0.5) (layer B.Cu) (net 14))
 (segment (start 216.1 103.93) (end 215.01 105.02) (width 0.5) (layer B.Cu) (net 14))
 (segment (start 213.23 121.3) (end 213.23 122.59) (width 0.5) (layer B.Cu) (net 14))
 (segment (start 215.8 118.82) (end 213.23 121.3) (width 0.5) (layer B.Cu) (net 14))
 (segment (start 215.8 115.81) (end 215.8 118.82) (width 0.5) (layer B.Cu) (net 14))
 (segment (start 215.48 115.58) (end 215.8 115.81) (width 0.5) (layer B.Cu) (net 14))
 (segment (start 210.99 115.58) (end 215.48 115.58) (width 0.5) (layer B.Cu) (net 14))
 (segment (start 210.44 115.09) (end 210.99 115.58) (width 0.5) (layer B.Cu) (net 14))
 (segment (start 210.44 112.15) (end 210.44 115.09) (width 0.5) (layer B.Cu) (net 14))
 (segment (start 212.28 110.35) (end 210.44 112.15) (width 0.5) (layer B.Cu) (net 14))
 (segment (start 216.1 103.93) (end 219.16 103.93) (width 0.5) (layer B.Cu) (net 14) (status 20))
 (segment (start 216.1 103.93) (end 222.99 103.93) (width 0.5) (layer B.Cu) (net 14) (status 20))
 (segment (start 223.09 104.03) (end 222.99 103.93) (width 0.5) (layer B.Cu) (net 14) (status 30))
 (segment (start 223.09 104.03) (end 223.03 103.97) (width 0.5) (layer B.Cu) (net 14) (status 30))
 (segment (start 223.09 104.03) (end 226.44 104.27) (width 1) (layer B.Cu) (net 14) (status 30))
 (segment (start 216.39 106.32) (end 219.95 106.32) (width 0.5) (layer B.Cu) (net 15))
 (segment (start 220.24 106.03) (end 223.09 106.03) (width 0.5) (layer B.Cu) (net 15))
 (segment (start 219.95 106.32) (end 220.24 106.03) (width 0.5) (layer B.Cu) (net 15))
 (segment (start 216.68 106.03) (end 216.39 106.32) (width 0.5) (layer B.Cu) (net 15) (status 30))
 (segment (start 223.09 106.03) (end 222.86 106.26) (width 0.5) (layer B.Cu) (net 15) (status 30))
 (segment (start 223.09 106.03) (end 226.44 106.81) (width 1) (layer B.Cu) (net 15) (status 30))
 (segment (start 225.47 106.81) (end 226.44 106.81) (width 0.5) (layer B.Cu) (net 15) (status 30))
 (segment (start 223.09 108.03) (end 220.77 108.03) (width 0.5) (layer B.Cu) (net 16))
 (segment (start 219.73 109.07) (end 219.73 110.18) (width 0.5) (layer B.Cu) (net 16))
 (segment (start 220.77 108.03) (end 219.73 109.07) (width 0.5) (layer B.Cu) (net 16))
 (segment (start 223.09 108.03) (end 226.44 109.35) (width 1) (layer B.Cu) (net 16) (status 30))
 (segment (start 225.99 109.35) (end 226.44 109.35) (width 0.5) (layer B.Cu) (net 16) (status 30))
 (segment (start 207.09 108.03) (end 203.58 109.35) (width 1) (layer B.Cu) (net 2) (status 30))
 (segment (start 204.35 109.35) (end 203.58 109.35) (width 0.5) (layer B.Cu) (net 2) (status 30))
 (segment (start 207.09 106.03) (end 203.58 106.81) (width 1) (layer B.Cu) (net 3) (status 30))
 (segment (start 207.09 104.03) (end 203.58 104.27) (width 1) (layer B.Cu) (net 4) (status 30))
 (segment (start 210.26 101.29) (end 209.52 102.03) (width 0.5) (layer B.Cu) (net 5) (status 10))
 (segment (start 209.52 102.03) (end 207.09 102.03) (width 0.5) (layer B.Cu) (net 5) (status 20))
 (segment (start 207.09 102.03) (end 208.42 102.03) (width 0.25) (layer B.Cu) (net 5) (status 30))
 (segment (start 207.09 102.03) (end 203.58 101.73) (width 1) (layer B.Cu) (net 5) (status 30))
 (segment (start 207.09 100.03) (end 207.1 100.04) (width 0.5) (layer B.Cu) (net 6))
 (segment (start 207.1 100.04) (end 211.73 100.04) (width 0.5) (layer B.Cu) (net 6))
 (segment (start 212.9 101.21) (end 214.72 101.21) (width 0.5) (layer B.Cu) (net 6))
 (segment (start 211.73 100.04) (end 212.9 101.21) (width 0.5) (layer B.Cu) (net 6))
 (segment (start 207.09 100.03) (end 203.58 99.19) (width 1) (layer B.Cu) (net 6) (status 30))
 (segment (start 207.09 98.03) (end 203.58 96.65) (width 1) (layer B.Cu) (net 7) (status 30))
 (segment (start 219.69 133.94) (end 219.69 130.77) (width 0.5) (layer B.Cu) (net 10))
 (segment (start 219.4 107.36) (end 219.34 117.31) (width 0.25) (layer F.Cu) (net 10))
 (segment (start 219.34 117.31) (end 220.63 125.8) (width 0.25) (layer F.Cu) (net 10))
 (segment (start 220.63 125.8) (end 219.69 130.77) (width 0.25) (layer F.Cu) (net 10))
 (via (at 219.69 130.77) (size 2) (drill 0.6) (layers F.Cu B.Cu) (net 10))
 (via (at 218 96.05) (size 2) (drill 0.6) (layers F.Cu B.Cu) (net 10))
 (segment (start 219.4 107.36) (end 218 96.05) (width 0.25) (layer F.Cu) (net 10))
 (segment (start 219.69 133.94) (end 219.61 134.02) (width 0.5) (layer B.Cu) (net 10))
 (segment (start 223.09 96.03) (end 218.01 96.04) (width 0.5) (layer B.Cu) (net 10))
 (segment (start 223.09 96.03) (end 226.44 94.11) (width 1) (layer B.Cu) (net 10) (status 30)))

